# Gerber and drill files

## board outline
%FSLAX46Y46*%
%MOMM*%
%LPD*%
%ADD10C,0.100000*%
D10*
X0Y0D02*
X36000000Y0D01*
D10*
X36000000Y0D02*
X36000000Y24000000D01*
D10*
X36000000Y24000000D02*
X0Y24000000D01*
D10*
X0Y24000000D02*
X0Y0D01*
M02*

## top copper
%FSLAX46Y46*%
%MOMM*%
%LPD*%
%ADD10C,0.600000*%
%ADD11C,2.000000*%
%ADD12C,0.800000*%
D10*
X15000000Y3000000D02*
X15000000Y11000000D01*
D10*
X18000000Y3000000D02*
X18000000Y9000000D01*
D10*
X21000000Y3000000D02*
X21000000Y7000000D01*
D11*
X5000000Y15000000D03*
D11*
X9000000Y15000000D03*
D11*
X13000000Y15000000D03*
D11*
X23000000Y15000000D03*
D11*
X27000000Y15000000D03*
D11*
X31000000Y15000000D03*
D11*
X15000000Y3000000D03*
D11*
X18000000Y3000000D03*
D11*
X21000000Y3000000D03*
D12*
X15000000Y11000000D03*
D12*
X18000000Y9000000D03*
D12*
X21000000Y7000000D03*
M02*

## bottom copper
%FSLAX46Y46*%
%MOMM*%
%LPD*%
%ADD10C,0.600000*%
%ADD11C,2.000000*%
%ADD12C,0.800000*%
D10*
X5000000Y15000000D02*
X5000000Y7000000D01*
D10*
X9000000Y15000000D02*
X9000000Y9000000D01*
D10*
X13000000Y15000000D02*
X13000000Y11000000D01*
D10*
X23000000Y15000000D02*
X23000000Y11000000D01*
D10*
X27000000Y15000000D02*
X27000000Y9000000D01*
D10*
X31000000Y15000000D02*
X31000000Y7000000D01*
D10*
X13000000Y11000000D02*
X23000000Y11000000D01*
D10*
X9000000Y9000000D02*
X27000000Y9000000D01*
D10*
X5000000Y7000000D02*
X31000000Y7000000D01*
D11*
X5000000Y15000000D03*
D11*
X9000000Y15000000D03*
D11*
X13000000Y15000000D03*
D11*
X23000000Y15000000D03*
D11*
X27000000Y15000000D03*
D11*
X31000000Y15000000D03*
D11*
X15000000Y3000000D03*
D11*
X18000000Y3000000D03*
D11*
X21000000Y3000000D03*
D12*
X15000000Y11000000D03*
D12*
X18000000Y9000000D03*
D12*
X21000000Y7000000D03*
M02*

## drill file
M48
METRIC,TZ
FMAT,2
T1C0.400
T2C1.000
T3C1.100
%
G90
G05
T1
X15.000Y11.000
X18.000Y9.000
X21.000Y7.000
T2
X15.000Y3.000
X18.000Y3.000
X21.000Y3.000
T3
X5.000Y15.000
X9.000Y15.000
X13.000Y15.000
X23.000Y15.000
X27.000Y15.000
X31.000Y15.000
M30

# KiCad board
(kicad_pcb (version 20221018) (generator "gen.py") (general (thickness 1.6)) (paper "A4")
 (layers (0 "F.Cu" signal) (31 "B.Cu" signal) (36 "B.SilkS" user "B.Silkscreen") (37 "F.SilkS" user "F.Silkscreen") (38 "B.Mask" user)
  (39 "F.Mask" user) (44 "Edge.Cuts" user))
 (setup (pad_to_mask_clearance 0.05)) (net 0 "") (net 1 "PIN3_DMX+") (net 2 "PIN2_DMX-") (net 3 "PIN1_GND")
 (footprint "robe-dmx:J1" (layer "F.Cu") (at 0 0)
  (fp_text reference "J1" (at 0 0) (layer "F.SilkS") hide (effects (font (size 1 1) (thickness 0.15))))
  (pad "3" thru_hole circle (at 5.0 9.0) (size 2.0 2.0) (drill 1.1) (layers "*.Cu" "*.Mask") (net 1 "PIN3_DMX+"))
  (pad "2" thru_hole circle (at 9.0 9.0) (size 2.0 2.0) (drill 1.1) (layers "*.Cu" "*.Mask") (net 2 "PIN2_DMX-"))
  (pad "1" thru_hole circle (at 13.0 9.0) (size 2.0 2.0) (drill 1.1) (layers "*.Cu" "*.Mask") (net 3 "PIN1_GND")))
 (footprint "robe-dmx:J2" (layer "F.Cu") (at 0 0)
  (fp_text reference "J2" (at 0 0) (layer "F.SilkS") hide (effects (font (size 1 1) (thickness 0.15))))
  (pad "1" thru_hole circle (at 23.0 9.0) (size 2.0 2.0) (drill 1.1) (layers "*.Cu" "*.Mask") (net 3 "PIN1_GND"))
  (pad "2" thru_hole circle (at 27.0 9.0) (size 2.0 2.0) (drill 1.1) (layers "*.Cu" "*.Mask") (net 2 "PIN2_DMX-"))
  (pad "3" thru_hole circle (at 31.0 9.0) (size 2.0 2.0) (drill 1.1) (layers "*.Cu" "*.Mask") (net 1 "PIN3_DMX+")))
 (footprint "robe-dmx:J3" (layer "F.Cu") (at 0 0)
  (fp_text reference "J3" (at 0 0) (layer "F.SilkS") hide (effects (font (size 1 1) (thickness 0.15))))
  (pad "1" thru_hole circle (at 15.0 21.0) (size 2.0 2.0) (drill 1.0) (layers "*.Cu" "*.Mask") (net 3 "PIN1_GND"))
  (pad "2" thru_hole circle (at 18.0 21.0) (size 2.0 2.0) (drill 1.0) (layers "*.Cu" "*.Mask") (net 2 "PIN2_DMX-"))
  (pad "3" thru_hole circle (at 21.0 21.0) (size 2.0 2.0) (drill 1.0) (layers "*.Cu" "*.Mask") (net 1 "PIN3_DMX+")))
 (segment (start 5.0 9.0) (end 5.0 17.0) (width 0.6) (layer "B.Cu") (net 1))
 (segment (start 9.0 9.0) (end 9.0 15.0) (width 0.6) (layer "B.Cu") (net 2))
 (segment (start 13.0 9.0) (end 13.0 13.0) (width 0.6) (layer "B.Cu") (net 3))
 (segment (start 23.0 9.0) (end 23.0 13.0) (width 0.6) (layer "B.Cu") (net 3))
 (segment (start 27.0 9.0) (end 27.0 15.0) (width 0.6) (layer "B.Cu") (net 2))
 (segment (start 31.0 9.0) (end 31.0 17.0) (width 0.6) (layer "B.Cu") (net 1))
 (segment (start 13.0 13.0) (end 23.0 13.0) (width 0.6) (layer "B.Cu") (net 3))
 (segment (start 9.0 15.0) (end 27.0 15.0) (width 0.6) (layer "B.Cu") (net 2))
 (segment (start 5.0 17.0) (end 31.0 17.0) (width 0.6) (layer "B.Cu") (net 1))
 (segment (start 15.0 21.0) (end 15.0 13.0) (width 0.6) (layer "F.Cu") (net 3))
 (segment (start 18.0 21.0) (end 18.0 15.0) (width 0.6) (layer "F.Cu") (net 2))
 (segment (start 21.0 21.0) (end 21.0 17.0) (width 0.6) (layer "F.Cu") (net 1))
 (via (at 15.0 13.0) (size 0.8) (drill 0.4) (layers "F.Cu" "B.Cu") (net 3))
 (via (at 18.0 15.0) (size 0.8) (drill 0.4) (layers "F.Cu" "B.Cu") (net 2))
 (via (at 21.0 17.0) (size 0.8) (drill 0.4) (layers "F.Cu" "B.Cu") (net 1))
 (gr_line (start 0 24.0) (end 36.0 24.0) (layer "Edge.Cuts") (width 0.1))
 (gr_line (start 36.0 24.0) (end 36.0 0.0) (layer "Edge.Cuts") (width 0.1))
 (gr_line (start 36.0 0.0) (end 0 0.0) (layer "Edge.Cuts") (width 0.1))
 (gr_line (start 0 0.0) (end 0 24.0) (layer "Edge.Cuts") (width 0.1)))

